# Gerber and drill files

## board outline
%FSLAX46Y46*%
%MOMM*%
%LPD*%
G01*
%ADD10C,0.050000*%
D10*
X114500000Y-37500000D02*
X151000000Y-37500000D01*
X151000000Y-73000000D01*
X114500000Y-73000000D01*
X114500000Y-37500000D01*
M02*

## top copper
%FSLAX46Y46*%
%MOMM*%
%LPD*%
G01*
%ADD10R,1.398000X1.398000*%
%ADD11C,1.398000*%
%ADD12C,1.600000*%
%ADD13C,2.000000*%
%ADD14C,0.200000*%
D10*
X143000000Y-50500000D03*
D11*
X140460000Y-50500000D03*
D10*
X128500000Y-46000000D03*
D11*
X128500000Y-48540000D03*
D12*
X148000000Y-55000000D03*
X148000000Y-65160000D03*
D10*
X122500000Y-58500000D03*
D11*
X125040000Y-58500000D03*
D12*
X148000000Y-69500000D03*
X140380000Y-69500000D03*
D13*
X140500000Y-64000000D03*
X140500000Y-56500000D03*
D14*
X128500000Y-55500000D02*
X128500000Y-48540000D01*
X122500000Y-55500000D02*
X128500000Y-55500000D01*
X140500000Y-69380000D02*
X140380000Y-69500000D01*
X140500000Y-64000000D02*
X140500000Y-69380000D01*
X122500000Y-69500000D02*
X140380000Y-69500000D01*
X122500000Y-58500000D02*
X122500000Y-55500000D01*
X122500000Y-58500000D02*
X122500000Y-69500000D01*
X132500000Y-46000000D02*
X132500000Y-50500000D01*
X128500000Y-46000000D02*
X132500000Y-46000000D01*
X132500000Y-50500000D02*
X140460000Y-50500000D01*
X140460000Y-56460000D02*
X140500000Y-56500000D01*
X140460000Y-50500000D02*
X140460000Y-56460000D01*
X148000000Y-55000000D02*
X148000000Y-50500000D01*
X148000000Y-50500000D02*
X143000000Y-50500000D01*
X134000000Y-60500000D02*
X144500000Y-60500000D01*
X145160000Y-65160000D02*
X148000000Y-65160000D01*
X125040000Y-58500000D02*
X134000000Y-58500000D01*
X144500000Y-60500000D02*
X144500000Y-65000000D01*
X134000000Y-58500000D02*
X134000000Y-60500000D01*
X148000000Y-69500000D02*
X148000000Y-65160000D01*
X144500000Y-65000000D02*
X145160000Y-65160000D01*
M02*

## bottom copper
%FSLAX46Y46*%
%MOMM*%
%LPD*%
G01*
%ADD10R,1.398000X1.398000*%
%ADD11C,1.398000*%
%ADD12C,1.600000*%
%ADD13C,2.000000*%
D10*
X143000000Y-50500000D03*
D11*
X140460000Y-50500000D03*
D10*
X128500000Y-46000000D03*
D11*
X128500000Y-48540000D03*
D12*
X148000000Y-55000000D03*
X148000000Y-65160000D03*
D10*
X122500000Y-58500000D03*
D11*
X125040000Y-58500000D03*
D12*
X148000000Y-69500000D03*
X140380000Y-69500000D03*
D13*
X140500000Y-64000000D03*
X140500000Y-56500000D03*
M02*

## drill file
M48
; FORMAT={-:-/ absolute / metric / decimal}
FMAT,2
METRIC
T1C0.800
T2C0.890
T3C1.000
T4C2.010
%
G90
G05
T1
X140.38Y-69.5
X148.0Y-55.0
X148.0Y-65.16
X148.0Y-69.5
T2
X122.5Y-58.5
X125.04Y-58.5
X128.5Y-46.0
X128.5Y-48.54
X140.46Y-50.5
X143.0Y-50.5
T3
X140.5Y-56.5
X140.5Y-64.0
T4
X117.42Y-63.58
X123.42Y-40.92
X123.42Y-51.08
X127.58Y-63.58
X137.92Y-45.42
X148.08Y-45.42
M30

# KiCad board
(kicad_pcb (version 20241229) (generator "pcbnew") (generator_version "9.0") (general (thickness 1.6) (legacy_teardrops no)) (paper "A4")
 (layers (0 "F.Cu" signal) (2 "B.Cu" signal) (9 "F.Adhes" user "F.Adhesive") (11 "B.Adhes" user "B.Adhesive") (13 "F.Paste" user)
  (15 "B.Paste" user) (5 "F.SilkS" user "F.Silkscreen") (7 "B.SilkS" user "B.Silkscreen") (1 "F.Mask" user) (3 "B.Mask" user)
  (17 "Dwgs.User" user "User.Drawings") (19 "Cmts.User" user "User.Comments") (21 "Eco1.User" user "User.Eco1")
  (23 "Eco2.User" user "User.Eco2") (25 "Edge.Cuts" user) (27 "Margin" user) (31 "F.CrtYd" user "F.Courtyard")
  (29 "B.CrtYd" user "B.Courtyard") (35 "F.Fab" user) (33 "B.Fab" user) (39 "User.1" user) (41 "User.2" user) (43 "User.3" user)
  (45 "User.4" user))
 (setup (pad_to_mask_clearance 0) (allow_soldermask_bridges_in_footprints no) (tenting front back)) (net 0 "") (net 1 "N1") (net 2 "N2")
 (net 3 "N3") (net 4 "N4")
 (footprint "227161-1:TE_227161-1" (layer "F.Cu") (at 143 50.5)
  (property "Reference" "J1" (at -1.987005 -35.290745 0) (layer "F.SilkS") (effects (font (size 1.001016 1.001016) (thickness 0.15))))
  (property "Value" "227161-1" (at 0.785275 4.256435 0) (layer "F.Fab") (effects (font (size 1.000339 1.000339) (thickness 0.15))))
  (pad "" np_thru_hole circle (at -5.08 -5.08) (size 2.01 2.01) (drill 2.01) (layers "*.Cu" "*.Mask"))
  (pad "" np_thru_hole circle (at 5.08 -5.08) (size 2.01 2.01) (drill 2.01) (layers "*.Cu" "*.Mask"))
  (pad "1" thru_hole rect (at 0 0) (size 1.398 1.398) (drill 0.89) (layers "*.Cu" "*.Mask") (remove_unused_layers no) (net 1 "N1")
   (solder_mask_margin 0.102))
  (pad "2" thru_hole circle (at -2.54 0) (size 1.398 1.398) (drill 0.89) (layers "*.Cu" "*.Mask") (remove_unused_layers no) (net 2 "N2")
   (solder_mask_margin 0.102)))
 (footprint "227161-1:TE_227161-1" (layer "F.Cu") (at 128.5 46 90)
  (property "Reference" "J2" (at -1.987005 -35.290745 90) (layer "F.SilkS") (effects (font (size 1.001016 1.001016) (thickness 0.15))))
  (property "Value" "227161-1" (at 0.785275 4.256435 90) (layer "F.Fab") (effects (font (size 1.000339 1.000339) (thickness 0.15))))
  (pad "" np_thru_hole circle (at -5.08 -5.08 90) (size 2.01 2.01) (drill 2.01) (layers "*.Cu" "*.Mask"))
  (pad "" np_thru_hole circle (at 5.08 -5.08 90) (size 2.01 2.01) (drill 2.01) (layers "*.Cu" "*.Mask"))
  (pad "1" thru_hole rect (at 0 0 90) (size 1.398 1.398) (drill 0.89) (layers "*.Cu" "*.Mask") (remove_unused_layers no) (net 2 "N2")
   (solder_mask_margin 0.102))
  (pad "2" thru_hole circle (at -2.54 0 90) (size 1.398 1.398) (drill 0.89) (layers "*.Cu" "*.Mask") (remove_unused_layers no) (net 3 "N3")
   (solder_mask_margin 0.102)))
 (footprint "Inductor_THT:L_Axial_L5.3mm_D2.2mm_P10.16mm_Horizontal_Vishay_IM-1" (layer "F.Cu") (at 148 55 -90)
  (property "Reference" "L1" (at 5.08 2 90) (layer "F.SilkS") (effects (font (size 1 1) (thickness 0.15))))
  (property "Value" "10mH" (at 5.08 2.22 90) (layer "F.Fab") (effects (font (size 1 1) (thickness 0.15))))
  (pad "1" thru_hole circle (at 0 0 270) (size 1.6 1.6) (drill 0.8) (layers "*.Cu" "*.Mask") (remove_unused_layers no) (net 1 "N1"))
  (pad "2" thru_hole circle (at 10.16 0 270) (size 1.6 1.6) (drill 0.8) (layers "*.Cu" "*.Mask") (remove_unused_layers no) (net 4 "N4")))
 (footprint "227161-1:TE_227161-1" (layer "F.Cu") (at 122.5 58.5 180)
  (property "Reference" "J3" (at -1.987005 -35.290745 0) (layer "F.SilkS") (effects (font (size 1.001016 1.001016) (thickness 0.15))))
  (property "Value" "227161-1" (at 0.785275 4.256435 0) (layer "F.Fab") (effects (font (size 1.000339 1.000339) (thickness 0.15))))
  (pad "" np_thru_hole circle (at -5.08 -5.08 180) (size 2.01 2.01) (drill 2.01) (layers "*.Cu" "*.Mask"))
  (pad "" np_thru_hole circle (at 5.08 -5.08 180) (size 2.01 2.01) (drill 2.01) (layers "*.Cu" "*.Mask"))
  (pad "1" thru_hole rect (at 0 0 180) (size 1.398 1.398) (drill 0.89) (layers "*.Cu" "*.Mask") (remove_unused_layers no) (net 3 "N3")
   (solder_mask_margin 0.102))
  (pad "2" thru_hole circle (at -2.54 0 180) (size 1.398 1.398) (drill 0.89) (layers "*.Cu" "*.Mask") (remove_unused_layers no) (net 4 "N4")
   (solder_mask_margin 0.102)))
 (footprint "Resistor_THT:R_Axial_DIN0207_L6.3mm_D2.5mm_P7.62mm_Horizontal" (layer "F.Cu") (at 148 69.5 180)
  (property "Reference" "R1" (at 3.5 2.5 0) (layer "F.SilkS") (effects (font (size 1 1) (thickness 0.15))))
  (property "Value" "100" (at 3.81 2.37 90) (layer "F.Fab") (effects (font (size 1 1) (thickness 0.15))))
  (pad "1" thru_hole circle (at 0 0 180) (size 1.6 1.6) (drill 0.8) (layers "*.Cu" "*.Mask") (remove_unused_layers no) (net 4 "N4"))
  (pad "2" thru_hole circle (at 7.62 0 180) (size 1.6 1.6) (drill 0.8) (layers "*.Cu" "*.Mask") (remove_unused_layers no) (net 3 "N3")))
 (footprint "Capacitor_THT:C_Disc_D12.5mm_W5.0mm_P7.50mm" (layer "F.Cu") (at 140.5 64 90)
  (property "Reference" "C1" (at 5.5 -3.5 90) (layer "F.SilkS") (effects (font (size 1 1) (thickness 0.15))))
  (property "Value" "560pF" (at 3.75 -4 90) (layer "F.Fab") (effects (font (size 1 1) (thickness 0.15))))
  (pad "1" thru_hole circle (at 0 0 90) (size 2 2) (drill 1) (layers "*.Cu" "*.Mask") (remove_unused_layers no) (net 3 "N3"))
  (pad "2" thru_hole circle (at 7.5 0 90) (size 2 2) (drill 1) (layers "*.Cu" "*.Mask") (remove_unused_layers no) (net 2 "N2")))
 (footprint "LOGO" (layer "B.Cu") (at 133 57.5 180)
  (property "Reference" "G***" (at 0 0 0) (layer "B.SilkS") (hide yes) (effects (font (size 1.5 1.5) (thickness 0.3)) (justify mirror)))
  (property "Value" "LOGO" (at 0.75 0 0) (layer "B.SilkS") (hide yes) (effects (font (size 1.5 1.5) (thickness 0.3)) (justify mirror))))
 (gr_poly (pts (xy 114.5 37.5) (xy 151 37.5) (xy 151 73) (xy 114.5 73)) (stroke (width 0.05) (type solid)) (fill no) (layer "Edge.Cuts"))
 (segment (start 128.5 55.5) (end 128.5 48.54) (width 0.2) (layer "F.Cu") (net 3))
 (segment (start 122.5 55.5) (end 128.5 55.5) (width 0.2) (layer "F.Cu") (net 3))
 (segment (start 140.5 69.38) (end 140.38 69.5) (width 0.2) (layer "F.Cu") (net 3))
 (segment (start 140.5 64) (end 140.5 69.38) (width 0.2) (layer "F.Cu") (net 3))
 (segment (start 122.5 69.5) (end 140.38 69.5) (width 0.2) (layer "F.Cu") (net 3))
 (segment (start 122.5 58.5) (end 122.5 55.5) (width 0.2) (layer "F.Cu") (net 3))
 (segment (start 122.5 58.5) (end 122.5 69.5) (width 0.2) (layer "F.Cu") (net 3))
 (segment (start 132.5 46) (end 132.5 50.5) (width 0.2) (layer "F.Cu") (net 2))
 (segment (start 128.5 46) (end 132.5 46) (width 0.2) (layer "F.Cu") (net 2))
 (segment (start 132.5 50.5) (end 140.46 50.5) (width 0.2) (layer "F.Cu") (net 2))
 (segment (start 140.46 56.46) (end 140.5 56.5) (width 0.2) (layer "F.Cu") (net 2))
 (segment (start 140.46 50.5) (end 140.46 56.46) (width 0.2) (layer "F.Cu") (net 2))
 (segment (start 148 55) (end 148 50.5) (width 0.2) (layer "F.Cu") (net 1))
 (segment (start 148 50.5) (end 143 50.5) (width 0.2) (layer "F.Cu") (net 1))
 (segment (start 134 60.5) (end 144.5 60.5) (width 0.2) (layer "F.Cu") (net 4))
 (segment (start 145.16 65.16) (end 148 65.16) (width 0.2) (layer "F.Cu") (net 4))
 (segment (start 125.04 58.5) (end 134 58.5) (width 0.2) (layer "F.Cu") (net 4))
 (segment (start 144.5 60.5) (end 144.5 65) (width 0.2) (layer "F.Cu") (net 4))
 (segment (start 134 58.5) (end 134 60.5) (width 0.2) (layer "F.Cu") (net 4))
 (segment (start 148 69.5) (end 148 65.16) (width 0.2) (layer "F.Cu") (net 4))
 (segment (start 144.5 65) (end 145.16 65.16) (width 0.2) (layer "F.Cu") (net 4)))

